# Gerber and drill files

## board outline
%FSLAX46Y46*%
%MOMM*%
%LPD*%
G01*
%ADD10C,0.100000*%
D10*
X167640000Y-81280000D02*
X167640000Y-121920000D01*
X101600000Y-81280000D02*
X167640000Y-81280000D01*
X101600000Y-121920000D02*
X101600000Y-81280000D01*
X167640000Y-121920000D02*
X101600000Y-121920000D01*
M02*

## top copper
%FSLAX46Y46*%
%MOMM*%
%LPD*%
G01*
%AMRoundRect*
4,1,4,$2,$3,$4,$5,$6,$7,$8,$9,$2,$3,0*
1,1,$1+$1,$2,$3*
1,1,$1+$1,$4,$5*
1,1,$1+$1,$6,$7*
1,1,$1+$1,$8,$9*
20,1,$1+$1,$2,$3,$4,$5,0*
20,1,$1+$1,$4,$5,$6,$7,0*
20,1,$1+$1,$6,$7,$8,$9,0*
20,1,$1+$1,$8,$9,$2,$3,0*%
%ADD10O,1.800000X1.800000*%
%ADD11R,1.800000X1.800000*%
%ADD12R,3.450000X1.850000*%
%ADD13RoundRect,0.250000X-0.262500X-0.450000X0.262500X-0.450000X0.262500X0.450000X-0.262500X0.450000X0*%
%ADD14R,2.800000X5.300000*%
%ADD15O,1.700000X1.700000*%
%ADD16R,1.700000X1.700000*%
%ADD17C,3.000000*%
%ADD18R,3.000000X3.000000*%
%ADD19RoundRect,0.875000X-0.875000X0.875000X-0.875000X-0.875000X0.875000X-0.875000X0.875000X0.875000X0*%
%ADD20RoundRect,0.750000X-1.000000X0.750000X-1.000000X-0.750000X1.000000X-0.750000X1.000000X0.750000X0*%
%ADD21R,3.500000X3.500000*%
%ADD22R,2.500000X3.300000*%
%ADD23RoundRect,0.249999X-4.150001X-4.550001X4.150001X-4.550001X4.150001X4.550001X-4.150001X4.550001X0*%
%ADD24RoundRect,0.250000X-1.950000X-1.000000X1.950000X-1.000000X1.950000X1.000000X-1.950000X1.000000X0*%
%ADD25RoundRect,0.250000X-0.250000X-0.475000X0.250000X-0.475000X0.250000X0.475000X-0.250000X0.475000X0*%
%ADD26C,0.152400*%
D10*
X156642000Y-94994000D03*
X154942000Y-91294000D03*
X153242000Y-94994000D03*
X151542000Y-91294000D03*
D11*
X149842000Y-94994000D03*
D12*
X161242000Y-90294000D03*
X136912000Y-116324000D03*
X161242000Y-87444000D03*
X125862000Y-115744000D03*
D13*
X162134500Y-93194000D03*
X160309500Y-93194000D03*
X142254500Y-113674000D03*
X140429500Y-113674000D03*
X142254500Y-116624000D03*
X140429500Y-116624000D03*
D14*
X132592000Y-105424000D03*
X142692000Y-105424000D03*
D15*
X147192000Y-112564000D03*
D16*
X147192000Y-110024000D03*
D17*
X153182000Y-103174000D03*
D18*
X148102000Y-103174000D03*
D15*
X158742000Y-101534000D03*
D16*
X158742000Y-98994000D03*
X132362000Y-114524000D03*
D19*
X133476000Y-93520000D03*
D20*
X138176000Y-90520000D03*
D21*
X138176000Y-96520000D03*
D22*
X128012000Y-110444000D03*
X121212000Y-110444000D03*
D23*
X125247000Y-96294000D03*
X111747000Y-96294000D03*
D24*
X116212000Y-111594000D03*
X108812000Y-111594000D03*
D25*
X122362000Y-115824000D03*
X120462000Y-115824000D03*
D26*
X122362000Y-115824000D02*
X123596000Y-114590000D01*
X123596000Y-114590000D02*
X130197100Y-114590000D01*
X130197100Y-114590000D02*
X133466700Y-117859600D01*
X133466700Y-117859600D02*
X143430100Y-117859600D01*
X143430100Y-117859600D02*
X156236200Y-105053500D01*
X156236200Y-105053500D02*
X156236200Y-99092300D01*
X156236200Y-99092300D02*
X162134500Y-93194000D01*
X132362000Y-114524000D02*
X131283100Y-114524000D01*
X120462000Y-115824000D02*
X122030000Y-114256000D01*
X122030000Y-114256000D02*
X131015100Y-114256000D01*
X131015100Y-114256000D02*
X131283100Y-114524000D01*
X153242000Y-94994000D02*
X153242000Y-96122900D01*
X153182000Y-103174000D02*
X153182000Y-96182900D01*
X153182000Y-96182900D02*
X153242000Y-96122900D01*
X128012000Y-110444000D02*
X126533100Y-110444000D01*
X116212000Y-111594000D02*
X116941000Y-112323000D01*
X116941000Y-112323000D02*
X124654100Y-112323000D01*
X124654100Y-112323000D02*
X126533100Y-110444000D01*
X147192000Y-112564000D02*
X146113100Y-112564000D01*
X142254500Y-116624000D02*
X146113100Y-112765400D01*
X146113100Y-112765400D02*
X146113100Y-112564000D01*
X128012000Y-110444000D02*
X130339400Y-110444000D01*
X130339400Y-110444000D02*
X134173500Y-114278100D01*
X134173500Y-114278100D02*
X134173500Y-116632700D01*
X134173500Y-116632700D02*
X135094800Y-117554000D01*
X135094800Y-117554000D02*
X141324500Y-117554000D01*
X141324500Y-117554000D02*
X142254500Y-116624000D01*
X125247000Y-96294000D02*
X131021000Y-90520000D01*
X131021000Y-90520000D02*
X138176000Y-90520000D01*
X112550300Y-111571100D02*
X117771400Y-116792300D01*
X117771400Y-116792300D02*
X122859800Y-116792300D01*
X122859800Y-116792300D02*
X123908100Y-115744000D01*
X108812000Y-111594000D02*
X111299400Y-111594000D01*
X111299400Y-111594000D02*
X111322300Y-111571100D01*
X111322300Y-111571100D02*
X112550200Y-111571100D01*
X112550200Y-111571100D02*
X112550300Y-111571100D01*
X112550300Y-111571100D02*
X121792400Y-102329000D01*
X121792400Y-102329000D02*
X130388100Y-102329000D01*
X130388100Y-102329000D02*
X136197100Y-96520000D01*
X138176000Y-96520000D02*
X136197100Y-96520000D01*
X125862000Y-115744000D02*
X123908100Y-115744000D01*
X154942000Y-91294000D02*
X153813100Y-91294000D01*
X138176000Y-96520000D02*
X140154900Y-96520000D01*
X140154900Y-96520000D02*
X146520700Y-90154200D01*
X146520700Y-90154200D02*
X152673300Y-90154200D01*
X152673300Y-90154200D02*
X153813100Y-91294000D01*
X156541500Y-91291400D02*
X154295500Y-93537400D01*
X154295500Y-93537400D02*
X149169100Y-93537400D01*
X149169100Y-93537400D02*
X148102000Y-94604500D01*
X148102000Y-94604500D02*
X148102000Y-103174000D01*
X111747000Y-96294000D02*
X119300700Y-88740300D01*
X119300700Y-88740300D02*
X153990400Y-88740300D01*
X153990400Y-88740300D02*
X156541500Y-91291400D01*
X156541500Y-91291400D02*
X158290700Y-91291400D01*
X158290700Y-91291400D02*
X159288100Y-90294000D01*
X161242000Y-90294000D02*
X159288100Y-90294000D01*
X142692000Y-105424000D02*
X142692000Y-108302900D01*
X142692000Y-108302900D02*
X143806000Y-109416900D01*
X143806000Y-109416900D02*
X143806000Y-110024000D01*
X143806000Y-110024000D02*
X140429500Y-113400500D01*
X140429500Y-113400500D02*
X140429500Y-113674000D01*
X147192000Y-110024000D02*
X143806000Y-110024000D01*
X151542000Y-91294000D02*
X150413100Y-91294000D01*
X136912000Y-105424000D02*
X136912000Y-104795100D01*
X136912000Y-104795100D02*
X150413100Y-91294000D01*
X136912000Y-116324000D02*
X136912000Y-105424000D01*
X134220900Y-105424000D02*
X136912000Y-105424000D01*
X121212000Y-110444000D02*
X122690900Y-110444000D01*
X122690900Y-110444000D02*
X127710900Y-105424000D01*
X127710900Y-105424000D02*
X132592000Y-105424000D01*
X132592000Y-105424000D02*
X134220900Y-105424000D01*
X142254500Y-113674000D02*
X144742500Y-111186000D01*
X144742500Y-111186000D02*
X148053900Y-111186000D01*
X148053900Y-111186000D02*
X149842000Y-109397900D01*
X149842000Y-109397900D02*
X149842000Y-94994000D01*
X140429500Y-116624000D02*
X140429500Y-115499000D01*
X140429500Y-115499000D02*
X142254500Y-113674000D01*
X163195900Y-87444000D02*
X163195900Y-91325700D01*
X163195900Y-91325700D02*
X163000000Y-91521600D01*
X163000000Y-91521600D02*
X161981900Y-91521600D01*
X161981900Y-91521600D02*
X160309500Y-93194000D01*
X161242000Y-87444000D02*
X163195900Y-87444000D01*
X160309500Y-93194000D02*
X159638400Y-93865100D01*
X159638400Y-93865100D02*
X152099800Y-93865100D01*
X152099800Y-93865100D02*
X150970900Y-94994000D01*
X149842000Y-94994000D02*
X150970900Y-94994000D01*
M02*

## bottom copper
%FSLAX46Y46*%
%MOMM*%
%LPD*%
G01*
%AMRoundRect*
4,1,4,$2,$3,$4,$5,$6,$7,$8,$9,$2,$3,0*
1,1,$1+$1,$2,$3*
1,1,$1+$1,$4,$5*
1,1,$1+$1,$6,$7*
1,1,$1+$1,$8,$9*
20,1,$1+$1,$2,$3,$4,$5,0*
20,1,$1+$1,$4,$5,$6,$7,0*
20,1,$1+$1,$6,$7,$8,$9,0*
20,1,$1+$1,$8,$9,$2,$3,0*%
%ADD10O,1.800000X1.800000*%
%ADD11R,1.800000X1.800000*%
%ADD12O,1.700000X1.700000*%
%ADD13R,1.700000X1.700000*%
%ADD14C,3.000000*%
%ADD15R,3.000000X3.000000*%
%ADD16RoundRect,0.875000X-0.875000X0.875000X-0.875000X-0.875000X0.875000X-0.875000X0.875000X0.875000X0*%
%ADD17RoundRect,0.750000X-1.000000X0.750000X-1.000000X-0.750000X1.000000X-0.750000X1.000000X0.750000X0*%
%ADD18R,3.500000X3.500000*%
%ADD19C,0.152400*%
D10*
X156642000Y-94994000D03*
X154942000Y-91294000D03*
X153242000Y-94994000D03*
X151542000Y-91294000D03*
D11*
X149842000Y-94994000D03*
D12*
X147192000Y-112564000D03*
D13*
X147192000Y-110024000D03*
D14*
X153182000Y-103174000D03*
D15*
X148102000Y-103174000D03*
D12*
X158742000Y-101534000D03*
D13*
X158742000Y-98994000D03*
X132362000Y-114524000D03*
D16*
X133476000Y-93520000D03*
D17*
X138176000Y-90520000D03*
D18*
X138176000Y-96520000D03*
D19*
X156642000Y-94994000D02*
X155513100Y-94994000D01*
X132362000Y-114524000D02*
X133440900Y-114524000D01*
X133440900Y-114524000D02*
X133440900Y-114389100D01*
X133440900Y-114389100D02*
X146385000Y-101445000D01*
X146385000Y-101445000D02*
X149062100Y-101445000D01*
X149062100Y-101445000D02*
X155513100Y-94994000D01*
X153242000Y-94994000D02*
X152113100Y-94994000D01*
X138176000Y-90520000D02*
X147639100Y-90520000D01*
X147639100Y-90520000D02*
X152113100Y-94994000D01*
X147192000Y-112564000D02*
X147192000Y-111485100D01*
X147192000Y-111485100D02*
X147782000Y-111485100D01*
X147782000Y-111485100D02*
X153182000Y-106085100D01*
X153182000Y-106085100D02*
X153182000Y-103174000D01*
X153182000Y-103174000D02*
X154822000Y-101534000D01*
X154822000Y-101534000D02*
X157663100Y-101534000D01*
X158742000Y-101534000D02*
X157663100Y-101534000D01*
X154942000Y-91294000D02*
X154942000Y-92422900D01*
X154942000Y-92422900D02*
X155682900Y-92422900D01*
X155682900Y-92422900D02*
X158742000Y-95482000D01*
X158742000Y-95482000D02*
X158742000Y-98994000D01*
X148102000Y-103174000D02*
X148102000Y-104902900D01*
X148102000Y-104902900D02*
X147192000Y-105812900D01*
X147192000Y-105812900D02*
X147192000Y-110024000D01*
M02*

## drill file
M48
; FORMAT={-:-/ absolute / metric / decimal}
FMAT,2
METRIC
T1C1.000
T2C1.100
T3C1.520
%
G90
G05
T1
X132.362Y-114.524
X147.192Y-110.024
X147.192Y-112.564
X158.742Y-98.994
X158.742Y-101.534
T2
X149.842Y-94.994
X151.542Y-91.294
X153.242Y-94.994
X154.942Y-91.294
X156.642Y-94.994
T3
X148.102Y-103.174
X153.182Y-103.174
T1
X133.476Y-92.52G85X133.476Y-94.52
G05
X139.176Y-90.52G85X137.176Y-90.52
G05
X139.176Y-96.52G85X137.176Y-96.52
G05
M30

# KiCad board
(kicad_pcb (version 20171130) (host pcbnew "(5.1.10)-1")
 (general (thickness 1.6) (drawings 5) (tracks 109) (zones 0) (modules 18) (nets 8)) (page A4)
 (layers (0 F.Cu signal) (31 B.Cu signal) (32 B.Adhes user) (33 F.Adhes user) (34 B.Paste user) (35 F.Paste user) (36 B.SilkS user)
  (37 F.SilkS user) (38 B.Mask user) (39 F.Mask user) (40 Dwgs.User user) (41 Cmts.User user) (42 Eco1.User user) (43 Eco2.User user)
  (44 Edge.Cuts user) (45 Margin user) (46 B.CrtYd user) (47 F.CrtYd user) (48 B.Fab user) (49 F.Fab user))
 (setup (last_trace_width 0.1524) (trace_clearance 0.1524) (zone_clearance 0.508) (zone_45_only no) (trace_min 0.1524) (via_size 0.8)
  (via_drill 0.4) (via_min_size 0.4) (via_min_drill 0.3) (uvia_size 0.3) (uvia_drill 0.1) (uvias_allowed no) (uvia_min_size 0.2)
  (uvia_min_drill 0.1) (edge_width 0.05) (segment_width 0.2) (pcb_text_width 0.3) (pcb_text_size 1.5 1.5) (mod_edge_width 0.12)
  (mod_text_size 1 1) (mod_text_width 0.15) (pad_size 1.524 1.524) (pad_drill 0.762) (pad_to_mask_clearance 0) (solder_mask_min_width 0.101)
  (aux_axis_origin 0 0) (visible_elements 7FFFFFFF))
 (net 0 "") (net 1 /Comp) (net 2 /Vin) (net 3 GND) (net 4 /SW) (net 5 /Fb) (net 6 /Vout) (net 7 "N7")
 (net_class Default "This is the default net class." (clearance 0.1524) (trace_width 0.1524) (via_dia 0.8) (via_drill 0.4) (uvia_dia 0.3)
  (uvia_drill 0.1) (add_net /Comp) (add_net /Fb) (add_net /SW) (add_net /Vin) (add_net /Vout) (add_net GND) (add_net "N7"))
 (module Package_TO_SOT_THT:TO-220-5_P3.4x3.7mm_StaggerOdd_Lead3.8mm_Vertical (layer F.Cu) (at 149.842 94.994)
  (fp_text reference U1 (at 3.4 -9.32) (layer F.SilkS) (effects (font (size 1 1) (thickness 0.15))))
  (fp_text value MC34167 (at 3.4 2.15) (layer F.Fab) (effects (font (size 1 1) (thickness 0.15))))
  (pad 5 thru_hole oval (at 6.8 0) (size 1.8 1.8) (drill 1.1) (layers *.Cu *.Mask) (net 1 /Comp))
  (pad 4 thru_hole oval (at 5.1 -3.7) (size 1.8 1.8) (drill 1.1) (layers *.Cu *.Mask) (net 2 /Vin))
  (pad 3 thru_hole oval (at 3.4 0) (size 1.8 1.8) (drill 1.1) (layers *.Cu *.Mask) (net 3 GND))
  (pad 2 thru_hole oval (at 1.7 -3.7) (size 1.8 1.8) (drill 1.1) (layers *.Cu *.Mask) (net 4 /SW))
  (pad 1 thru_hole rect (at 0 0) (size 1.8 1.8) (drill 1.1) (layers *.Cu *.Mask) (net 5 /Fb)))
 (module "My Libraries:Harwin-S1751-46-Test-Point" (layer F.Cu) (at 161.242 90.294)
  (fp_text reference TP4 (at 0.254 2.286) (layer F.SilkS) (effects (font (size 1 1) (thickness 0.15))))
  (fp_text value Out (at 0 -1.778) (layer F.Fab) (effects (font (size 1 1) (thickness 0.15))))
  (pad 1 smd rect (at 0 0) (size 3.45 1.85) (layers F.Cu F.Paste F.Mask) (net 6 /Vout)))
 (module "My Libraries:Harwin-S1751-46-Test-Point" (layer F.Cu) (at 136.912 116.324)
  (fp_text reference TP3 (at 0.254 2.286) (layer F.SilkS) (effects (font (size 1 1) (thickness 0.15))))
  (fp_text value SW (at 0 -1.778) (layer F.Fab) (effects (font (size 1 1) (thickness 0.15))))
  (pad 1 smd rect (at 0 0) (size 3.45 1.85) (layers F.Cu F.Paste F.Mask) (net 4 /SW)))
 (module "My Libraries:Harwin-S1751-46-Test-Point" (layer F.Cu) (at 161.242 87.444)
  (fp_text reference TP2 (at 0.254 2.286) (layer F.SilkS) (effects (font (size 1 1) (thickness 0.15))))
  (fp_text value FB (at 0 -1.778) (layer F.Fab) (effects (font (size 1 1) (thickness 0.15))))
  (pad 1 smd rect (at 0 0) (size 3.45 1.85) (layers F.Cu F.Paste F.Mask) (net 5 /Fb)))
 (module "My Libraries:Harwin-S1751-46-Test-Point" (layer F.Cu) (at 125.862 115.744)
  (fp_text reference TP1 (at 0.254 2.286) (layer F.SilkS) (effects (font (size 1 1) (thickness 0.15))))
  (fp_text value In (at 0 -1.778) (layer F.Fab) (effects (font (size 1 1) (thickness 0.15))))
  (pad 1 smd rect (at 0 0) (size 3.45 1.85) (layers F.Cu F.Paste F.Mask) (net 2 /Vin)))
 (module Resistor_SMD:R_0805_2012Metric (layer F.Cu) (at 161.222 93.194)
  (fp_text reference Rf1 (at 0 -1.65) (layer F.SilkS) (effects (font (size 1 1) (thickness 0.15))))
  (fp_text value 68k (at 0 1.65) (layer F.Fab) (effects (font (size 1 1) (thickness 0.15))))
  (pad 2 smd roundrect (at 0.9125 0) (size 1.025 1.4) (layers F.Cu F.Paste F.Mask) (roundrect_rratio 0.243902) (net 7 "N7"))
  (pad 1 smd roundrect (at -0.9125 0) (size 1.025 1.4) (layers F.Cu F.Paste F.Mask) (roundrect_rratio 0.243902) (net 5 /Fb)))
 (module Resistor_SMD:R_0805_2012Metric (layer F.Cu) (at 141.342 113.674)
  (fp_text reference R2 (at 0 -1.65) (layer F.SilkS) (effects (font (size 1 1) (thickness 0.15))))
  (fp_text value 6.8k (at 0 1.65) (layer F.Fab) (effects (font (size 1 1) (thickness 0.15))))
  (pad 2 smd roundrect (at 0.9125 0) (size 1.025 1.4) (layers F.Cu F.Paste F.Mask) (roundrect_rratio 0.243902) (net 5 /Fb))
  (pad 1 smd roundrect (at -0.9125 0) (size 1.025 1.4) (layers F.Cu F.Paste F.Mask) (roundrect_rratio 0.243902) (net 6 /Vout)))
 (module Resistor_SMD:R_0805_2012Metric (layer F.Cu) (at 141.342 116.624)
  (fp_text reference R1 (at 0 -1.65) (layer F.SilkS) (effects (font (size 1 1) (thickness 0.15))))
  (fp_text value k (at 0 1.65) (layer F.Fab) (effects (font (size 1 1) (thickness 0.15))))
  (pad 2 smd roundrect (at 0.9125 0) (size 1.025 1.4) (layers F.Cu F.Paste F.Mask) (roundrect_rratio 0.243902) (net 3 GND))
  (pad 1 smd roundrect (at -0.9125 0) (size 1.025 1.4) (layers F.Cu F.Paste F.Mask) (roundrect_rratio 0.243902) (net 5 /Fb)))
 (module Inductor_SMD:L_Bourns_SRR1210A (layer F.Cu) (at 137.642 105.424)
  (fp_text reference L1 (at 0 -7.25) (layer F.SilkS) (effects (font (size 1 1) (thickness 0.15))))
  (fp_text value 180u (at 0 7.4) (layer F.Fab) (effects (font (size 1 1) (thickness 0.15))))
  (pad 1 smd rect (at -5.05 0) (size 2.8 5.3) (layers F.Cu F.Paste F.Mask) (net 4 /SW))
  (pad 2 smd rect (at 5.05 0) (size 2.8 5.3) (layers F.Cu F.Paste F.Mask) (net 6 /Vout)))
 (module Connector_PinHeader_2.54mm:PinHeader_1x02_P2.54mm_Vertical (layer F.Cu) (at 147.192 110.024)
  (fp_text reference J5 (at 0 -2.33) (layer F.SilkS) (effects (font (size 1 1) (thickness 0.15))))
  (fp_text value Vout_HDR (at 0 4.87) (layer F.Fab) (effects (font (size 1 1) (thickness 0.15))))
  (pad 2 thru_hole oval (at 0 2.54) (size 1.7 1.7) (drill 1) (layers *.Cu *.Mask) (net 3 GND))
  (pad 1 thru_hole rect (at 0 0) (size 1.7 1.7) (drill 1) (layers *.Cu *.Mask) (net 6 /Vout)))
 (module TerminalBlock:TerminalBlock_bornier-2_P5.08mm (layer F.Cu) (at 148.102 103.174)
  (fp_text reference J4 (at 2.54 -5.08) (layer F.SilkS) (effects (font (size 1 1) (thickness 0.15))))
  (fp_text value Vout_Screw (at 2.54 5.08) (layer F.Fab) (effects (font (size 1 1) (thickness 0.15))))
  (pad 2 thru_hole circle (at 5.08 0) (size 3 3) (drill 1.52) (layers *.Cu *.Mask) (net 3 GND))
  (pad 1 thru_hole rect (at 0 0) (size 3 3) (drill 1.52) (layers *.Cu *.Mask) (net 6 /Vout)))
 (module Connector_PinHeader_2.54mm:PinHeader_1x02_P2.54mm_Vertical (layer F.Cu) (at 158.742 98.994)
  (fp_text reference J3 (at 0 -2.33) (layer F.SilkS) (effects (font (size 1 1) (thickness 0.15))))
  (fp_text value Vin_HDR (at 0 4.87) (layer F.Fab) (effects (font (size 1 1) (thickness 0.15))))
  (pad 2 thru_hole oval (at 0 2.54) (size 1.7 1.7) (drill 1) (layers *.Cu *.Mask) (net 3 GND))
  (pad 1 thru_hole rect (at 0 0) (size 1.7 1.7) (drill 1) (layers *.Cu *.Mask) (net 2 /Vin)))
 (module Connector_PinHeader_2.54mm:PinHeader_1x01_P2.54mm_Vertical (layer F.Cu) (at 132.362 114.524)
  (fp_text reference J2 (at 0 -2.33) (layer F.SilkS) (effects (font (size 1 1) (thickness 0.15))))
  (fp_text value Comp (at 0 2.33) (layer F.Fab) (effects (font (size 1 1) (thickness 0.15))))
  (pad 1 thru_hole rect (at 0 0) (size 1.7 1.7) (drill 1) (layers *.Cu *.Mask) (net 1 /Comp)))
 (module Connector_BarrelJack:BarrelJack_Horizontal (layer F.Cu) (at 138.176 96.52 270)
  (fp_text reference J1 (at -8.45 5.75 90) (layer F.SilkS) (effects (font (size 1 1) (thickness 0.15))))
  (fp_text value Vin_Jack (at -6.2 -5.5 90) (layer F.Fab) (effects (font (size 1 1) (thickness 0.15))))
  (pad 3 thru_hole roundrect (at -3 4.7 270) (size 3.5 3.5) (drill oval 3 1) (layers *.Cu *.Mask) (roundrect_rratio 0.25))
  (pad 2 thru_hole roundrect (at -6 0 270) (size 3 3.5) (drill oval 1 3) (layers *.Cu *.Mask) (roundrect_rratio 0.25) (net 3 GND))
  (pad 1 thru_hole rect (at 0 0 270) (size 3.5 3.5) (drill oval 1 3) (layers *.Cu *.Mask) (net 2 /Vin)))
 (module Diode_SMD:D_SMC (layer F.Cu) (at 124.612 110.444)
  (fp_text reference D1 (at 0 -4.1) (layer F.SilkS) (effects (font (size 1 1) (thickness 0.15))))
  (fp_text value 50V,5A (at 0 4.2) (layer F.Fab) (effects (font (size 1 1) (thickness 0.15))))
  (pad 2 smd rect (at 3.4 0 90) (size 3.3 2.5) (layers F.Cu F.Paste F.Mask) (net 3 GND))
  (pad 1 smd rect (at -3.4 0 90) (size 3.3 2.5) (layers F.Cu F.Paste F.Mask) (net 4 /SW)))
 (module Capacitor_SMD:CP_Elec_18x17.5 (layer F.Cu) (at 118.497 96.294)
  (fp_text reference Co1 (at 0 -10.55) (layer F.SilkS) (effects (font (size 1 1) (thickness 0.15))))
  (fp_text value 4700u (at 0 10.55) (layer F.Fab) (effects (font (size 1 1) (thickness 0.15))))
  (pad 2 smd roundrect (at 6.75 0) (size 8.8 9.6) (layers F.Cu F.Paste F.Mask) (roundrect_rratio 0.028409) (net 3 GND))
  (pad 1 smd roundrect (at -6.75 0) (size 8.8 9.6) (layers F.Cu F.Paste F.Mask) (roundrect_rratio 0.028409) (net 6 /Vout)))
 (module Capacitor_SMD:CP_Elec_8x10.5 (layer F.Cu) (at 112.512 111.594)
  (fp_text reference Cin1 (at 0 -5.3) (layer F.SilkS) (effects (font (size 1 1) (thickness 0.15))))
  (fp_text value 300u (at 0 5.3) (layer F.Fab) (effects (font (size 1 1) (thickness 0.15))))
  (pad 2 smd roundrect (at 3.7 0) (size 4.4 2.5) (layers F.Cu F.Paste F.Mask) (roundrect_rratio 0.1) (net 3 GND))
  (pad 1 smd roundrect (at -3.7 0) (size 4.4 2.5) (layers F.Cu F.Paste F.Mask) (roundrect_rratio 0.1) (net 2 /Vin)))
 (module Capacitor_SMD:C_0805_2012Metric (layer F.Cu) (at 121.412 115.824)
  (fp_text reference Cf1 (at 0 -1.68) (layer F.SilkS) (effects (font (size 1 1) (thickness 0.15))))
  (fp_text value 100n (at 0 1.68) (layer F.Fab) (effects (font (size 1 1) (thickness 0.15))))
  (pad 2 smd roundrect (at 0.95 0) (size 1 1.45) (layers F.Cu F.Paste F.Mask) (roundrect_rratio 0.25) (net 7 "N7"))
  (pad 1 smd roundrect (at -0.95 0) (size 1 1.45) (layers F.Cu F.Paste F.Mask) (roundrect_rratio 0.25) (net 1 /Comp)))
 (gr_line (start 167.64 81.28) (end 167.64 121.92) (layer Edge.Cuts) (width 0.1))
 (gr_line (start 101.6 81.28) (end 167.64 81.28) (layer Edge.Cuts) (width 0.1))
 (gr_line (start 101.6 121.92) (end 101.6 81.28) (layer Edge.Cuts) (width 0.1))
 (gr_line (start 167.64 121.92) (end 101.6 121.92) (layer Edge.Cuts) (width 0.1))
 (segment (start 122.362 115.824) (end 123.596 114.59) (width 0.1524) (layer F.Cu) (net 7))
 (segment (start 123.596 114.59) (end 130.1971 114.59) (width 0.1524) (layer F.Cu) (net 7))
 (segment (start 130.1971 114.59) (end 133.4667 117.8596) (width 0.1524) (layer F.Cu) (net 7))
 (segment (start 133.4667 117.8596) (end 143.4301 117.8596) (width 0.1524) (layer F.Cu) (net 7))
 (segment (start 143.4301 117.8596) (end 156.2362 105.0535) (width 0.1524) (layer F.Cu) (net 7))
 (segment (start 156.2362 105.0535) (end 156.2362 99.0923) (width 0.1524) (layer F.Cu) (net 7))
 (segment (start 156.2362 99.0923) (end 162.1345 93.194) (width 0.1524) (layer F.Cu) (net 7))
 (segment (start 132.362 114.524) (end 131.2831 114.524) (width 0.1524) (layer F.Cu) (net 1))
 (segment (start 120.462 115.824) (end 122.03 114.256) (width 0.1524) (layer F.Cu) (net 1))
 (segment (start 122.03 114.256) (end 131.0151 114.256) (width 0.1524) (layer F.Cu) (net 1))
 (segment (start 131.0151 114.256) (end 131.2831 114.524) (width 0.1524) (layer F.Cu) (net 1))
 (segment (start 156.642 94.994) (end 155.5131 94.994) (width 0.1524) (layer B.Cu) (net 1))
 (segment (start 132.362 114.524) (end 133.4409 114.524) (width 0.1524) (layer B.Cu) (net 1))
 (segment (start 133.4409 114.524) (end 133.4409 114.3891) (width 0.1524) (layer B.Cu) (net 1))
 (segment (start 133.4409 114.3891) (end 146.385 101.445) (width 0.1524) (layer B.Cu) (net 1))
 (segment (start 146.385 101.445) (end 149.0621 101.445) (width 0.1524) (layer B.Cu) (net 1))
 (segment (start 149.0621 101.445) (end 155.5131 94.994) (width 0.1524) (layer B.Cu) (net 1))
 (segment (start 153.242 94.994) (end 153.242 96.1229) (width 0.1524) (layer F.Cu) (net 3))
 (segment (start 153.182 103.174) (end 153.182 96.1829) (width 0.1524) (layer F.Cu) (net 3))
 (segment (start 153.182 96.1829) (end 153.242 96.1229) (width 0.1524) (layer F.Cu) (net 3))
 (segment (start 153.242 94.994) (end 152.1131 94.994) (width 0.1524) (layer B.Cu) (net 3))
 (segment (start 138.176 90.52) (end 147.6391 90.52) (width 0.1524) (layer B.Cu) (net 3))
 (segment (start 147.6391 90.52) (end 152.1131 94.994) (width 0.1524) (layer B.Cu) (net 3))
 (segment (start 128.012 110.444) (end 126.5331 110.444) (width 0.1524) (layer F.Cu) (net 3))
 (segment (start 116.212 111.594) (end 116.941 112.323) (width 0.1524) (layer F.Cu) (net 3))
 (segment (start 116.941 112.323) (end 124.6541 112.323) (width 0.1524) (layer F.Cu) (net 3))
 (segment (start 124.6541 112.323) (end 126.5331 110.444) (width 0.1524) (layer F.Cu) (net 3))
 (segment (start 147.192 112.564) (end 146.1131 112.564) (width 0.1524) (layer F.Cu) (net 3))
 (segment (start 142.2545 116.624) (end 146.1131 112.7654) (width 0.1524) (layer F.Cu) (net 3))
 (segment (start 146.1131 112.7654) (end 146.1131 112.564) (width 0.1524) (layer F.Cu) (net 3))
 (segment (start 128.012 110.444) (end 130.3394 110.444) (width 0.1524) (layer F.Cu) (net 3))
 (segment (start 130.3394 110.444) (end 134.1735 114.2781) (width 0.1524) (layer F.Cu) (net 3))
 (segment (start 134.1735 114.2781) (end 134.1735 116.6327) (width 0.1524) (layer F.Cu) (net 3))
 (segment (start 134.1735 116.6327) (end 135.0948 117.554) (width 0.1524) (layer F.Cu) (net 3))
 (segment (start 135.0948 117.554) (end 141.3245 117.554) (width 0.1524) (layer F.Cu) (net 3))
 (segment (start 141.3245 117.554) (end 142.2545 116.624) (width 0.1524) (layer F.Cu) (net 3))
 (segment (start 125.247 96.294) (end 131.021 90.52) (width 0.1524) (layer F.Cu) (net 3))
 (segment (start 131.021 90.52) (end 138.176 90.52) (width 0.1524) (layer F.Cu) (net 3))
 (segment (start 147.192 112.564) (end 147.192 111.4851) (width 0.1524) (layer B.Cu) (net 3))
 (segment (start 147.192 111.4851) (end 147.782 111.4851) (width 0.1524) (layer B.Cu) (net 3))
 (segment (start 147.782 111.4851) (end 153.182 106.0851) (width 0.1524) (layer B.Cu) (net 3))
 (segment (start 153.182 106.0851) (end 153.182 103.174) (width 0.1524) (layer B.Cu) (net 3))
 (segment (start 153.182 103.174) (end 154.822 101.534) (width 0.1524) (layer B.Cu) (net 3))
 (segment (start 154.822 101.534) (end 157.6631 101.534) (width 0.1524) (layer B.Cu) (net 3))
 (segment (start 158.742 101.534) (end 157.6631 101.534) (width 0.1524) (layer B.Cu) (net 3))
 (segment (start 154.942 91.294) (end 154.942 92.4229) (width 0.1524) (layer B.Cu) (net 2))
 (segment (start 154.942 92.4229) (end 155.6829 92.4229) (width 0.1524) (layer B.Cu) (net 2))
 (segment (start 155.6829 92.4229) (end 158.742 95.482) (width 0.1524) (layer B.Cu) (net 2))
 (segment (start 158.742 95.482) (end 158.742 98.994) (width 0.1524) (layer B.Cu) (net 2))
 (segment (start 112.5503 111.5711) (end 117.7714 116.7923) (width 0.1524) (layer F.Cu) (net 2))
 (segment (start 117.7714 116.7923) (end 122.8598 116.7923) (width 0.1524) (layer F.Cu) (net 2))
 (segment (start 122.8598 116.7923) (end 123.9081 115.744) (width 0.1524) (layer F.Cu) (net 2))
 (segment (start 108.812 111.594) (end 111.2994 111.594) (width 0.1524) (layer F.Cu) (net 2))
 (segment (start 111.2994 111.594) (end 111.3223 111.5711) (width 0.1524) (layer F.Cu) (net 2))
 (segment (start 111.3223 111.5711) (end 112.5502 111.5711) (width 0.1524) (layer F.Cu) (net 2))
 (segment (start 112.5502 111.5711) (end 112.5503 111.5711) (width 0.1524) (layer F.Cu) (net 2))
 (segment (start 112.5503 111.5711) (end 121.7924 102.329) (width 0.1524) (layer F.Cu) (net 2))
 (segment (start 121.7924 102.329) (end 130.3881 102.329) (width 0.1524) (layer F.Cu) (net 2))
 (segment (start 130.3881 102.329) (end 136.1971 96.52) (width 0.1524) (layer F.Cu) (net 2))
 (segment (start 138.176 96.52) (end 136.1971 96.52) (width 0.1524) (layer F.Cu) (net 2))
 (segment (start 125.862 115.744) (end 123.9081 115.744) (width 0.1524) (layer F.Cu) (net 2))
 (segment (start 154.942 91.294) (end 153.8131 91.294) (width 0.1524) (layer F.Cu) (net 2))
 (segment (start 138.176 96.52) (end 140.1549 96.52) (width 0.1524) (layer F.Cu) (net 2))
 (segment (start 140.1549 96.52) (end 146.5207 90.1542) (width 0.1524) (layer F.Cu) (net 2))
 (segment (start 146.5207 90.1542) (end 152.6733 90.1542) (width 0.1524) (layer F.Cu) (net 2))
 (segment (start 152.6733 90.1542) (end 153.8131 91.294) (width 0.1524) (layer F.Cu) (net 2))
 (segment (start 148.102 103.174) (end 148.102 104.9029) (width 0.1524) (layer B.Cu) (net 6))
 (segment (start 148.102 104.9029) (end 147.192 105.8129) (width 0.1524) (layer B.Cu) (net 6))
 (segment (start 147.192 105.8129) (end 147.192 110.024) (width 0.1524) (layer B.Cu) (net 6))
 (segment (start 156.5415 91.2914) (end 154.2955 93.5374) (width 0.1524) (layer F.Cu) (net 6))
 (segment (start 154.2955 93.5374) (end 149.1691 93.5374) (width 0.1524) (layer F.Cu) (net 6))
 (segment (start 149.1691 93.5374) (end 148.102 94.6045) (width 0.1524) (layer F.Cu) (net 6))
 (segment (start 148.102 94.6045) (end 148.102 103.174) (width 0.1524) (layer F.Cu) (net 6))
 (segment (start 111.747 96.294) (end 119.3007 88.7403) (width 0.1524) (layer F.Cu) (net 6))
 (segment (start 119.3007 88.7403) (end 153.9904 88.7403) (width 0.1524) (layer F.Cu) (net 6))
 (segment (start 153.9904 88.7403) (end 156.5415 91.2914) (width 0.1524) (layer F.Cu) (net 6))
 (segment (start 156.5415 91.2914) (end 158.2907 91.2914) (width 0.1524) (layer F.Cu) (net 6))
 (segment (start 158.2907 91.2914) (end 159.2881 90.294) (width 0.1524) (layer F.Cu) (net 6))
 (segment (start 161.242 90.294) (end 159.2881 90.294) (width 0.1524) (layer F.Cu) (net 6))
 (segment (start 142.692 105.424) (end 142.692 108.3029) (width 0.1524) (layer F.Cu) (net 6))
 (segment (start 142.692 108.3029) (end 143.806 109.4169) (width 0.1524) (layer F.Cu) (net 6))
 (segment (start 143.806 109.4169) (end 143.806 110.024) (width 0.1524) (layer F.Cu) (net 6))
 (segment (start 143.806 110.024) (end 140.4295 113.4005) (width 0.1524) (layer F.Cu) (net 6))
 (segment (start 140.4295 113.4005) (end 140.4295 113.674) (width 0.1524) (layer F.Cu) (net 6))
 (segment (start 147.192 110.024) (end 143.806 110.024) (width 0.1524) (layer F.Cu) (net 6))
 (segment (start 151.542 91.294) (end 150.4131 91.294) (width 0.1524) (layer F.Cu) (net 4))
 (segment (start 136.912 105.424) (end 136.912 104.7951) (width 0.1524) (layer F.Cu) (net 4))
 (segment (start 136.912 104.7951) (end 150.4131 91.294) (width 0.1524) (layer F.Cu) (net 4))
 (segment (start 136.912 116.324) (end 136.912 105.424) (width 0.1524) (layer F.Cu) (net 4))
 (segment (start 134.2209 105.424) (end 136.912 105.424) (width 0.1524) (layer F.Cu) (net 4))
 (segment (start 121.212 110.444) (end 122.6909 110.444) (width 0.1524) (layer F.Cu) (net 4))
 (segment (start 122.6909 110.444) (end 127.7109 105.424) (width 0.1524) (layer F.Cu) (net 4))
 (segment (start 127.7109 105.424) (end 132.592 105.424) (width 0.1524) (layer F.Cu) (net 4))
 (segment (start 132.592 105.424) (end 134.2209 105.424) (width 0.1524) (layer F.Cu) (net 4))
 (segment (start 142.2545 113.674) (end 144.7425 111.186) (width 0.1524) (layer F.Cu) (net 5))
 (segment (start 144.7425 111.186) (end 148.0539 111.186) (width 0.1524) (layer F.Cu) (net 5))
 (segment (start 148.0539 111.186) (end 149.842 109.3979) (width 0.1524) (layer F.Cu) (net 5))
 (segment (start 149.842 109.3979) (end 149.842 94.994) (width 0.1524) (layer F.Cu) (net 5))
 (segment (start 140.4295 116.624) (end 140.4295 115.499) (width 0.1524) (layer F.Cu) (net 5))
 (segment (start 140.4295 115.499) (end 142.2545 113.674) (width 0.1524) (layer F.Cu) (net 5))
 (segment (start 163.1959 87.444) (end 163.1959 91.3257) (width 0.1524) (layer F.Cu) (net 5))
 (segment (start 163.1959 91.3257) (end 163 91.5216) (width 0.1524) (layer F.Cu) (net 5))
 (segment (start 163 91.5216) (end 161.9819 91.5216) (width 0.1524) (layer F.Cu) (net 5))
 (segment (start 161.9819 91.5216) (end 160.3095 93.194) (width 0.1524) (layer F.Cu) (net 5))
 (segment (start 161.242 87.444) (end 163.1959 87.444) (width 0.1524) (layer F.Cu) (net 5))
 (segment (start 160.3095 93.194) (end 159.6384 93.8651) (width 0.1524) (layer F.Cu) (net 5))
 (segment (start 159.6384 93.8651) (end 152.0998 93.8651) (width 0.1524) (layer F.Cu) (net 5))
 (segment (start 152.0998 93.8651) (end 150.9709 94.994) (width 0.1524) (layer F.Cu) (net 5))
 (segment (start 149.842 94.994) (end 150.9709 94.994) (width 0.1524) (layer F.Cu) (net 5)))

